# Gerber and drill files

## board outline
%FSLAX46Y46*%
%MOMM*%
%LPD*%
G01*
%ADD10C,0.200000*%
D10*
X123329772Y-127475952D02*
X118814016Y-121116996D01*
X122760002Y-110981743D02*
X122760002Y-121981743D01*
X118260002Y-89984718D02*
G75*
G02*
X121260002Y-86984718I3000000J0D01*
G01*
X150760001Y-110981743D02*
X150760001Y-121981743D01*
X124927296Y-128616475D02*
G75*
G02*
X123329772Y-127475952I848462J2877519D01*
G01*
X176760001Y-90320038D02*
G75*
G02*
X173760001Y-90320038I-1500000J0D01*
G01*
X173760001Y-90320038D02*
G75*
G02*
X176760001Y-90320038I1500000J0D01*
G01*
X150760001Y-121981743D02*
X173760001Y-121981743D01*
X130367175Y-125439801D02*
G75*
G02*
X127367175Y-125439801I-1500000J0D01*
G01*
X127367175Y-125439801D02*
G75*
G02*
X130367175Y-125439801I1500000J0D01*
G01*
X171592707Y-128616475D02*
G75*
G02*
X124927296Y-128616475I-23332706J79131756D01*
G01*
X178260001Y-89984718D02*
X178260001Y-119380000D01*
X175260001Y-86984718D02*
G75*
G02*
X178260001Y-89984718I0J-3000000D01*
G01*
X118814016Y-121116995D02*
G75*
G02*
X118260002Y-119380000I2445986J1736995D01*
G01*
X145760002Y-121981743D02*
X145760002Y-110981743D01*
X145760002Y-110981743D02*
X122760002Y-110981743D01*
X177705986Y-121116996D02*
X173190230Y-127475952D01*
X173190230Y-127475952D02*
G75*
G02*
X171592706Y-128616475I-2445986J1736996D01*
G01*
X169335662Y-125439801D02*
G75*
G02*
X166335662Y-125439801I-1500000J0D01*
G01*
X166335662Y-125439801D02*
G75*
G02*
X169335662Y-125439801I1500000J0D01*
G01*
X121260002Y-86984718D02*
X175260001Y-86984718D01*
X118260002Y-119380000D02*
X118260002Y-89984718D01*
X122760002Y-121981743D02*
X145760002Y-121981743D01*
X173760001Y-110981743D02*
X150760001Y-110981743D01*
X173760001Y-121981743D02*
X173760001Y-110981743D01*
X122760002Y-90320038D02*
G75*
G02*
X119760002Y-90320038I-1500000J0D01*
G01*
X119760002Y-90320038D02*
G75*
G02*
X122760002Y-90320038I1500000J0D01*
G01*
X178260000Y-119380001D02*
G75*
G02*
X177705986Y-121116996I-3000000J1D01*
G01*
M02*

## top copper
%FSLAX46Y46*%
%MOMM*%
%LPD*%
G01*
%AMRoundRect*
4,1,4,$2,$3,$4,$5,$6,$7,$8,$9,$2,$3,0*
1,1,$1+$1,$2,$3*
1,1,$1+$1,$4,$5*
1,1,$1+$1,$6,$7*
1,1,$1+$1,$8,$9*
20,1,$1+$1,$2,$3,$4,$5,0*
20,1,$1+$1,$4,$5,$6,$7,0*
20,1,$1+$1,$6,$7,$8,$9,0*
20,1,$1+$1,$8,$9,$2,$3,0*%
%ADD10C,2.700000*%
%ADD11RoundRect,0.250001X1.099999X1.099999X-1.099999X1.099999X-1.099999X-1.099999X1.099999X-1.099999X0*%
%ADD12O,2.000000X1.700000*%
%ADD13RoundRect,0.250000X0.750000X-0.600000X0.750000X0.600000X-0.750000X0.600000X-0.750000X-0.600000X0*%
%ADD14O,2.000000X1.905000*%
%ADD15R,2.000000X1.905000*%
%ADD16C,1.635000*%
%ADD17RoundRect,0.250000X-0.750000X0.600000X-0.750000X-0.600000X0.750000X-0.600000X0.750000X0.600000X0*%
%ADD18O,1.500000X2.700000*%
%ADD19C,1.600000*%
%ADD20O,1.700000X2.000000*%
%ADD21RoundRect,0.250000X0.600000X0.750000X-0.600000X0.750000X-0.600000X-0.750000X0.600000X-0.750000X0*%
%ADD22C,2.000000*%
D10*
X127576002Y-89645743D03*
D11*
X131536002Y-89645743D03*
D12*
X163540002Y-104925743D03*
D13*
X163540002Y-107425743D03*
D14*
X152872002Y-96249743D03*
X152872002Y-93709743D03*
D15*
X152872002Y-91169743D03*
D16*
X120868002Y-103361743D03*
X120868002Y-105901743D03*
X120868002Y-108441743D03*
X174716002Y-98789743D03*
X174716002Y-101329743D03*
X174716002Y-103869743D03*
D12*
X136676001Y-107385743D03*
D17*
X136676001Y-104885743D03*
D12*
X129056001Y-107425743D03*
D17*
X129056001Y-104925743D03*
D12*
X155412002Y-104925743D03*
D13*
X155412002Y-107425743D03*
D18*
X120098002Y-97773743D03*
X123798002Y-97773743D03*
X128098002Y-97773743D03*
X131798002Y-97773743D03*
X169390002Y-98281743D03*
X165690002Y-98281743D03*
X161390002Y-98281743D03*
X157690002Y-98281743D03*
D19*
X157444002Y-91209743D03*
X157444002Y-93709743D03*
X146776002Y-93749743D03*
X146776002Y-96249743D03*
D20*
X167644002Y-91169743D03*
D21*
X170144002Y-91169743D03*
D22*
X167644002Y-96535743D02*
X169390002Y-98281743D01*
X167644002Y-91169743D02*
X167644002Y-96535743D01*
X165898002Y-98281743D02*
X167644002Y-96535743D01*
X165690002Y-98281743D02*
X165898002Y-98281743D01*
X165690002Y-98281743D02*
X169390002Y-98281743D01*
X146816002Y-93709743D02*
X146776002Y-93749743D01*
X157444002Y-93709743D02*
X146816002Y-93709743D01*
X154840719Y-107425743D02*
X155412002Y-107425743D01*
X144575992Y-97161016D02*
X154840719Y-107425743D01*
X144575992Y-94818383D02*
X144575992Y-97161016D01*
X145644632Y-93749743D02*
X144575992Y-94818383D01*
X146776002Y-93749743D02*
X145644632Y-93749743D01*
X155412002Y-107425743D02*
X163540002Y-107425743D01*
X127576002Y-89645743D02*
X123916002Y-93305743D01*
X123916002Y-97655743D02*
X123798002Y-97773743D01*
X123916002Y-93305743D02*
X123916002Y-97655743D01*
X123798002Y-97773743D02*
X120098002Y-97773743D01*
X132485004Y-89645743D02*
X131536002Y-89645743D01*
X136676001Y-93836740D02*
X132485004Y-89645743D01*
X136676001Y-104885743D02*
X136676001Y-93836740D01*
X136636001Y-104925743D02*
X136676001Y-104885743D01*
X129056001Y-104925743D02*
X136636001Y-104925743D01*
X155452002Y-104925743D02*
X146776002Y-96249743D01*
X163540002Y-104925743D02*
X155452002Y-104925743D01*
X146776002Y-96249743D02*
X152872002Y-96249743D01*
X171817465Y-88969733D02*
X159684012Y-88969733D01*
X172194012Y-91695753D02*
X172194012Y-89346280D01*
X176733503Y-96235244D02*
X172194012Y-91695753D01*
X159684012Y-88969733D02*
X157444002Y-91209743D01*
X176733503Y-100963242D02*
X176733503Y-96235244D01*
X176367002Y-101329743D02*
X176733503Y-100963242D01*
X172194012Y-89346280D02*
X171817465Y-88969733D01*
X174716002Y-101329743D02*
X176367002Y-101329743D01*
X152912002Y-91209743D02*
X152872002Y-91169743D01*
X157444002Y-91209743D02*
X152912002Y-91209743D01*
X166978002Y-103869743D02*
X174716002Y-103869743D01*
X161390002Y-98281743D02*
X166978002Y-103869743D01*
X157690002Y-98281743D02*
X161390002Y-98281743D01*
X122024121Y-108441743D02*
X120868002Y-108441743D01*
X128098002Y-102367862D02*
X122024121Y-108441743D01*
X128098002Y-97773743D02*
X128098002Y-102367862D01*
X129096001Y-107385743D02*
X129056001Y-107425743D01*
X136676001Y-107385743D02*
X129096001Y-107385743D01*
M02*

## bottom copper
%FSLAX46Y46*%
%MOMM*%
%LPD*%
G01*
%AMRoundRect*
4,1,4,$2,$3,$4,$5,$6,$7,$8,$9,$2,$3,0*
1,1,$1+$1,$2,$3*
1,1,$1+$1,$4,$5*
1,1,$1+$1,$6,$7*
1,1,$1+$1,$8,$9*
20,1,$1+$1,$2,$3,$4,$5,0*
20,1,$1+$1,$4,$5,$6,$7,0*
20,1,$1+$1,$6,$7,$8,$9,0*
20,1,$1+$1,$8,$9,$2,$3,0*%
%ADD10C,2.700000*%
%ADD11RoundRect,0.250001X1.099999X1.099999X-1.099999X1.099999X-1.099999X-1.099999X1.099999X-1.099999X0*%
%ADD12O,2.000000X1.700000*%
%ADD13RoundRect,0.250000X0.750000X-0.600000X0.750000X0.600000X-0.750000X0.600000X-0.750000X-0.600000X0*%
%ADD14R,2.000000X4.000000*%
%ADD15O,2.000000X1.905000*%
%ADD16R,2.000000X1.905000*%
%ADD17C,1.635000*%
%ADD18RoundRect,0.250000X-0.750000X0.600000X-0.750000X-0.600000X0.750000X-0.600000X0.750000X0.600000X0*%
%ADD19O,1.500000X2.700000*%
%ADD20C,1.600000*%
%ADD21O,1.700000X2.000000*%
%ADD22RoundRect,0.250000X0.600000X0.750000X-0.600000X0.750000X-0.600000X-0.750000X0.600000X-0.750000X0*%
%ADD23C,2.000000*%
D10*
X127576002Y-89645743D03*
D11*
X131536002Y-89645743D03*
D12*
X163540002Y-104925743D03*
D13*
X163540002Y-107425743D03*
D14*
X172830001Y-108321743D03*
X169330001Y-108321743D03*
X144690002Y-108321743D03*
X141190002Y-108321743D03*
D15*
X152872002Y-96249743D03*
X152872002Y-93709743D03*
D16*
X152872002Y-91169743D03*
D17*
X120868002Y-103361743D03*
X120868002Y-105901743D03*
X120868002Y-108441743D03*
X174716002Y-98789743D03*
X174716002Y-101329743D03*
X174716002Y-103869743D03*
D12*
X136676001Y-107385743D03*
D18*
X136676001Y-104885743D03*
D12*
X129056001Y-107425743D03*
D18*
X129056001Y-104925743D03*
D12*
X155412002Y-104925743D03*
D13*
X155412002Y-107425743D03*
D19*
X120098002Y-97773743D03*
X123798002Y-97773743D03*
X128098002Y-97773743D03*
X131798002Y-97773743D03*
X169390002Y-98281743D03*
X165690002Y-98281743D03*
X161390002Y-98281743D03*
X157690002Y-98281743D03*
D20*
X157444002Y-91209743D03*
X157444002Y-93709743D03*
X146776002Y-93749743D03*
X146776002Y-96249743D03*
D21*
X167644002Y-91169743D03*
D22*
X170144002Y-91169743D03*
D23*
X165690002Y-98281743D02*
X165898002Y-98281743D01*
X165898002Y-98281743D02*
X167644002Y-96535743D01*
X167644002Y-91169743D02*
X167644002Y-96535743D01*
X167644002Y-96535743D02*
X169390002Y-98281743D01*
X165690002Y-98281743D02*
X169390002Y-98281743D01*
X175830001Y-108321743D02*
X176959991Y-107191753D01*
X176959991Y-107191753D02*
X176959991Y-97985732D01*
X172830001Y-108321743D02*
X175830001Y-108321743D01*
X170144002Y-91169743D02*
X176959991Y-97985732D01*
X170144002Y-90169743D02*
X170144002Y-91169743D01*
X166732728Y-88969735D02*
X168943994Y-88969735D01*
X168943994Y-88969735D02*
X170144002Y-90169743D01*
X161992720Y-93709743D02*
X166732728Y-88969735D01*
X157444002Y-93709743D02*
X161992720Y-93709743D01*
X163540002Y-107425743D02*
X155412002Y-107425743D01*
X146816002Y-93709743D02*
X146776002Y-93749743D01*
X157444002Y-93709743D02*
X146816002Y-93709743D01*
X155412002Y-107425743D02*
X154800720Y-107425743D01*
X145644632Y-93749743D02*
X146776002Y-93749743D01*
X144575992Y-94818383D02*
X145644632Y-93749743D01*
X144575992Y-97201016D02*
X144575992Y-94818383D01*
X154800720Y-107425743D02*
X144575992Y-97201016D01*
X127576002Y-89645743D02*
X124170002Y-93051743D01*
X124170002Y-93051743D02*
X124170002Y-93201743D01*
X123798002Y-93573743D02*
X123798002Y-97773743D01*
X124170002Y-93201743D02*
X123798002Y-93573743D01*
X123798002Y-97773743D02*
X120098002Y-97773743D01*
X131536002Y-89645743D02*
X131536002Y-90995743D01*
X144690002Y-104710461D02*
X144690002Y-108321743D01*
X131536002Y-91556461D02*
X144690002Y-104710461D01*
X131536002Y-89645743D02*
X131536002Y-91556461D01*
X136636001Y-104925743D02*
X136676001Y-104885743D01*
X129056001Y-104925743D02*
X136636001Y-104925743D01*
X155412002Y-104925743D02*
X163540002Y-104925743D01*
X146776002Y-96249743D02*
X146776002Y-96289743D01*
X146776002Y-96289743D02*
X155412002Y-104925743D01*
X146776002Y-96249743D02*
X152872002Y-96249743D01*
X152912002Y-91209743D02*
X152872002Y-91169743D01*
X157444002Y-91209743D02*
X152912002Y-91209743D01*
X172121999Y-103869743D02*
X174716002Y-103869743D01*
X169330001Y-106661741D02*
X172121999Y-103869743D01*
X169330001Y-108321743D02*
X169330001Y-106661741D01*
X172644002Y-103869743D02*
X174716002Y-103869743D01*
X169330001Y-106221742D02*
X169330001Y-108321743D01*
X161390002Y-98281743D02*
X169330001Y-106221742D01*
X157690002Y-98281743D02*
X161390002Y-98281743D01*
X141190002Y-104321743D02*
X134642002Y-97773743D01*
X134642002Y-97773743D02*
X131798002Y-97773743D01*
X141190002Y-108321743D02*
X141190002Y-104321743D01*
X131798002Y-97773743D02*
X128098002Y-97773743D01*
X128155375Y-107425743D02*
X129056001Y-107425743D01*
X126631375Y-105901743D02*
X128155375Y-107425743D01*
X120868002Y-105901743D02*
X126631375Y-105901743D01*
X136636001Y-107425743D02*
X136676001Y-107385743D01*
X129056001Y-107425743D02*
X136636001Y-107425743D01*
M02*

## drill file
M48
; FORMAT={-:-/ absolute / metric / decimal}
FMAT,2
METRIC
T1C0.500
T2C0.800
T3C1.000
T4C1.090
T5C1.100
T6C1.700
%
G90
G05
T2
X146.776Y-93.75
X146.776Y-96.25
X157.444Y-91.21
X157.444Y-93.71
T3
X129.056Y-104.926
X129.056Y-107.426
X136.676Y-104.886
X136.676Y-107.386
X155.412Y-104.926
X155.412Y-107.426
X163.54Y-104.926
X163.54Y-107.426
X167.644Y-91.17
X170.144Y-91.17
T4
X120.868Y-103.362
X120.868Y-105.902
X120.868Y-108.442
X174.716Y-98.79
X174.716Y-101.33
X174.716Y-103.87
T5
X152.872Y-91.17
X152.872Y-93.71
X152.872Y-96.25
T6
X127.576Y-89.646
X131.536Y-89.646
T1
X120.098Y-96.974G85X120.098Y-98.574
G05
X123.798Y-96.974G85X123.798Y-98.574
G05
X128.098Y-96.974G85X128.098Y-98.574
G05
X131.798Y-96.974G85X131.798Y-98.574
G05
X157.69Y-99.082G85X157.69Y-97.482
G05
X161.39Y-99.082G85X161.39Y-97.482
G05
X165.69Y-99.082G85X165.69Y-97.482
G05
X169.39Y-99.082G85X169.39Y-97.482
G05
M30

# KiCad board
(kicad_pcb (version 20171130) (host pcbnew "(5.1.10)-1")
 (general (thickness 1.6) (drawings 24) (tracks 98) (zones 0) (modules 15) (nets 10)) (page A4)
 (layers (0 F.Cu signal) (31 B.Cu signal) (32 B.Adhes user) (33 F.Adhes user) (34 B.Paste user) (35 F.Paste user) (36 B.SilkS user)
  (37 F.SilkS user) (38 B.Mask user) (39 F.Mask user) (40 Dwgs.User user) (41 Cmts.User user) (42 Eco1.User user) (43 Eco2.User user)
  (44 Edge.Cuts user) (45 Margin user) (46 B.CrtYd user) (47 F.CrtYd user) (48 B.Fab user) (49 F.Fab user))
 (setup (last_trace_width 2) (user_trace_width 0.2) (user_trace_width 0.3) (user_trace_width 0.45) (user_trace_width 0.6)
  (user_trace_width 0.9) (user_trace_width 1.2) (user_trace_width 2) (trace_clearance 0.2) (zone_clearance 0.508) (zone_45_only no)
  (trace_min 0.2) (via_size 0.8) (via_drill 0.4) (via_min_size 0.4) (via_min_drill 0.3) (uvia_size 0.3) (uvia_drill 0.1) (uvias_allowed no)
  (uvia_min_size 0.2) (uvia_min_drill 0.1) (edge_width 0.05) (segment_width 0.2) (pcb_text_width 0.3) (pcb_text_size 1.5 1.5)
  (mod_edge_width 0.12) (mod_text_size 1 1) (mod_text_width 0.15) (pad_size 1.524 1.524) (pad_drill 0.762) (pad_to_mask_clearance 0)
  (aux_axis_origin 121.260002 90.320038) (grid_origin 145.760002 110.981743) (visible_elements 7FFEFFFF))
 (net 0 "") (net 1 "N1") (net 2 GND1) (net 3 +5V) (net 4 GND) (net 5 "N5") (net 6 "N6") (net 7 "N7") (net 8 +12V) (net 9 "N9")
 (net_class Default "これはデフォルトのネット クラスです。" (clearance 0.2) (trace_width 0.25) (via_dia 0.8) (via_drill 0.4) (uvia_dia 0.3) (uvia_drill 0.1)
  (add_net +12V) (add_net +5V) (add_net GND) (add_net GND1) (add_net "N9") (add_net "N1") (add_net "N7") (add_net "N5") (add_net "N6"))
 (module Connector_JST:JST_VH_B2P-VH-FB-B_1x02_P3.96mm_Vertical (layer F.Cu) (at 131.536002 89.645743 180)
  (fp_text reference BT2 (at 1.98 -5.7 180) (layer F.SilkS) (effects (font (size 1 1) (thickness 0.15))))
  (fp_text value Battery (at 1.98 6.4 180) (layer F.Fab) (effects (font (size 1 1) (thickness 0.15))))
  (pad 2 thru_hole circle (at 3.96 0 180) (size 2.7 2.7) (drill 1.7) (layers *.Cu *.Mask) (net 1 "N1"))
  (pad 1 thru_hole roundrect (at 0 0 180) (size 2.7 2.7) (drill 1.7) (layers *.Cu *.Mask) (roundrect_rratio 0.09259299999999999)
   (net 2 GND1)))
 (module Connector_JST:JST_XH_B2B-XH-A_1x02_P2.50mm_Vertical (layer F.Cu) (at 163.540002 107.425743 90)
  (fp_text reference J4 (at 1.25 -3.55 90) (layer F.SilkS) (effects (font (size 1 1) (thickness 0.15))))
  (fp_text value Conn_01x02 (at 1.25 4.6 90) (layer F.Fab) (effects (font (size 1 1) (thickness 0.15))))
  (pad 2 thru_hole oval (at 2.5 0 90) (size 1.7 2) (drill 1) (layers *.Cu *.Mask) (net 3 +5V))
  (pad 1 thru_hole roundrect (at 0 0 90) (size 1.7 2) (drill 1) (layers *.Cu *.Mask) (roundrect_rratio 0.147059) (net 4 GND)))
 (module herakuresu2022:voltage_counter (layer F.Cu) (at 162.330001 111.821743)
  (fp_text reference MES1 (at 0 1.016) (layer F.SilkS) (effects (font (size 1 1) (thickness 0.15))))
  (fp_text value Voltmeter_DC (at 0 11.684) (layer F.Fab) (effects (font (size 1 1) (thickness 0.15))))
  (pad 1 smd rect (at 10.5 -3.5) (size 2 4) (layers B.Cu B.Paste B.Mask) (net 4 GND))
  (pad 2 smd rect (at 7 -3.5) (size 2 4) (layers B.Cu B.Paste B.Mask) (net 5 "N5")))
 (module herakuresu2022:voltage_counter (layer F.Cu) (at 134.190002 111.821743)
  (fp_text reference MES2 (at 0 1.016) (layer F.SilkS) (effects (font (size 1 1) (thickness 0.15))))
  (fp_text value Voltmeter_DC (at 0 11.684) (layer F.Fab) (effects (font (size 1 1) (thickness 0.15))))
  (pad 1 smd rect (at 10.5 -3.5) (size 2 4) (layers B.Cu B.Paste B.Mask) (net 2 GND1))
  (pad 2 smd rect (at 7 -3.5) (size 2 4) (layers B.Cu B.Paste B.Mask) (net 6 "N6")))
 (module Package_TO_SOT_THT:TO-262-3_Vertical (layer F.Cu) (at 152.872002 91.169743 270)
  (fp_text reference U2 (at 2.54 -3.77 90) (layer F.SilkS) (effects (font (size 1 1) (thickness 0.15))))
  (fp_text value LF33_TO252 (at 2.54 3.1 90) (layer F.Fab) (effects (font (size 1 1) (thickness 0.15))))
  (pad 3 thru_hole oval (at 5.08 0 270) (size 1.905 2) (drill 1.1) (layers *.Cu *.Mask) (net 3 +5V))
  (pad 2 thru_hole oval (at 2.54 0 270) (size 1.905 2) (drill 1.1) (layers *.Cu *.Mask) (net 4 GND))
  (pad 1 thru_hole rect (at 0 0 270) (size 1.905 2) (drill 1.1) (layers *.Cu *.Mask) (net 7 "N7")))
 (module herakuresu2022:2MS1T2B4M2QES (layer F.Cu) (at 120.868002 108.441743)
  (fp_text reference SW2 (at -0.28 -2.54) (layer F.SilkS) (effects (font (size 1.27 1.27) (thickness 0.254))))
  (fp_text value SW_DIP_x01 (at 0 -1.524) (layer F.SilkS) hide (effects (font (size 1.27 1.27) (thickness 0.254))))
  (pad 3 thru_hole circle (at 0 -5.08) (size 1.635 1.635) (drill 1.09) (layers *.Cu *.Mask))
  (pad 2 thru_hole circle (at 0 -2.54) (size 1.635 1.635) (drill 1.09) (layers *.Cu *.Mask) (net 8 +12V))
  (pad 1 thru_hole circle (at 0 0) (size 1.635 1.635) (drill 1.09) (layers *.Cu *.Mask) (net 6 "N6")))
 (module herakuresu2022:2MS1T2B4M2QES (layer F.Cu) (at 174.716002 103.869743)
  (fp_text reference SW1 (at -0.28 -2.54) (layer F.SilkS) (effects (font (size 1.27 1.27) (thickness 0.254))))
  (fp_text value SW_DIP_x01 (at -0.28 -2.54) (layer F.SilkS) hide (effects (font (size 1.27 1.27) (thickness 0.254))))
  (pad 3 thru_hole circle (at 0 -5.08) (size 1.635 1.635) (drill 1.09) (layers *.Cu *.Mask))
  (pad 2 thru_hole circle (at 0 -2.54) (size 1.635 1.635) (drill 1.09) (layers *.Cu *.Mask) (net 7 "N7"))
  (pad 1 thru_hole circle (at 0 0) (size 1.635 1.635) (drill 1.09) (layers *.Cu *.Mask) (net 5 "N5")))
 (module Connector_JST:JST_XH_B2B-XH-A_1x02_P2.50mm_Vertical (layer F.Cu) (at 136.676001 104.885743 270)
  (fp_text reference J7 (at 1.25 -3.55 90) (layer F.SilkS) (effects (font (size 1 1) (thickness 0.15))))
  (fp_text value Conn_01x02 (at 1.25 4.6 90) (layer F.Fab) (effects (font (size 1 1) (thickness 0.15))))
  (pad 2 thru_hole oval (at 2.5 0 270) (size 1.7 2) (drill 1) (layers *.Cu *.Mask) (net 8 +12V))
  (pad 1 thru_hole roundrect (at 0 0 270) (size 1.7 2) (drill 1) (layers *.Cu *.Mask) (roundrect_rratio 0.147059) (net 2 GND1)))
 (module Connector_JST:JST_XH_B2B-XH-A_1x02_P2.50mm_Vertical (layer F.Cu) (at 129.056001 104.925743 270)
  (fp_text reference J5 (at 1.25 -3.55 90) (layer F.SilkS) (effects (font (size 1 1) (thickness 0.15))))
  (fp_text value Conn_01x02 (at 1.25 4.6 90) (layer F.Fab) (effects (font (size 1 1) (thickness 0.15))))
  (pad 2 thru_hole oval (at 2.5 0 270) (size 1.7 2) (drill 1) (layers *.Cu *.Mask) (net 8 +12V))
  (pad 1 thru_hole roundrect (at 0 0 270) (size 1.7 2) (drill 1) (layers *.Cu *.Mask) (roundrect_rratio 0.147059) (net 2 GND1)))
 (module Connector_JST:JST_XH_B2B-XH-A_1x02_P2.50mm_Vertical (layer F.Cu) (at 155.412002 107.425743 90)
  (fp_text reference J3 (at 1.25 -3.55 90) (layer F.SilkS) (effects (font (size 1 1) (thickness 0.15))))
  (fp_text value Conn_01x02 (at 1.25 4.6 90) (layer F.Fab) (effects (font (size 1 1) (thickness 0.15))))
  (pad 2 thru_hole oval (at 2.5 0 90) (size 1.7 2) (drill 1) (layers *.Cu *.Mask) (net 3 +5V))
  (pad 1 thru_hole roundrect (at 0 0 90) (size 1.7 2) (drill 1) (layers *.Cu *.Mask) (roundrect_rratio 0.147059) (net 4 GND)))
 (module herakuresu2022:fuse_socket (layer F.Cu) (at 125.948002 95.233743)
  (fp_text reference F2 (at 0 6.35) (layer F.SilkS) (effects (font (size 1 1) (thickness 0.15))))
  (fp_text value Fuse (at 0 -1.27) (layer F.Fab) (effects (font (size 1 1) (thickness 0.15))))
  (pad 1 thru_hole oval (at -5.85 2.54) (size 1.5 2.7) (drill oval 0.5 2.1) (layers *.Cu *.Mask) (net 1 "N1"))
  (pad 1 thru_hole oval (at -2.15 2.54) (size 1.5 2.7) (drill oval 0.5 2.1) (layers *.Cu *.Mask) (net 1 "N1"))
  (pad 2 thru_hole oval (at 2.15 2.54) (size 1.5 2.7) (drill oval 0.5 2.1) (layers *.Cu *.Mask) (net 6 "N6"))
  (pad 2 thru_hole oval (at 5.85 2.54) (size 1.5 2.7) (drill oval 0.5 2.1) (layers *.Cu *.Mask) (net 6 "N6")))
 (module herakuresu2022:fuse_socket (layer F.Cu) (at 163.540002 100.821743 180)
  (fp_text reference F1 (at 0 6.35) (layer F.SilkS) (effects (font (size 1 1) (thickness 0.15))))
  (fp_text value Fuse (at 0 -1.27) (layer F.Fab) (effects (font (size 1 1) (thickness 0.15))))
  (pad 1 thru_hole oval (at -5.85 2.54 180) (size 1.5 2.7) (drill oval 0.5 2.1) (layers *.Cu *.Mask) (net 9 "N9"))
  (pad 1 thru_hole oval (at -2.15 2.54 180) (size 1.5 2.7) (drill oval 0.5 2.1) (layers *.Cu *.Mask) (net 9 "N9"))
  (pad 2 thru_hole oval (at 2.15 2.54 180) (size 1.5 2.7) (drill oval 0.5 2.1) (layers *.Cu *.Mask) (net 5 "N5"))
  (pad 2 thru_hole oval (at 5.85 2.54 180) (size 1.5 2.7) (drill oval 0.5 2.1) (layers *.Cu *.Mask) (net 5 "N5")))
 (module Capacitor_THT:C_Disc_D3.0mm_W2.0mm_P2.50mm (layer F.Cu) (at 157.444002 93.709743 90)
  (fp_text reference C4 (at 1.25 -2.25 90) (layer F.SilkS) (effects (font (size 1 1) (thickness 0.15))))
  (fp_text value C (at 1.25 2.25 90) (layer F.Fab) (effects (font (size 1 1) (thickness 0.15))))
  (pad 2 thru_hole circle (at 2.5 0 90) (size 1.6 1.6) (drill 0.8) (layers *.Cu *.Mask) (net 7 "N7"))
  (pad 1 thru_hole circle (at 0 0 90) (size 1.6 1.6) (drill 0.8) (layers *.Cu *.Mask) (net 4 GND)))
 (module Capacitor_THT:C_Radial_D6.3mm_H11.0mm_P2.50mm (layer F.Cu) (at 146.776002 96.249743 90)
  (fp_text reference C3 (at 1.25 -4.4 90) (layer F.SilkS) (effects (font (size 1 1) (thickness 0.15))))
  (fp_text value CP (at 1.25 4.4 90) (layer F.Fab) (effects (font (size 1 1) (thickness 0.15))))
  (pad 2 thru_hole circle (at 2.5 0 90) (size 1.6 1.6) (drill 0.8) (layers *.Cu *.Mask) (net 4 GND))
  (pad 1 thru_hole circle (at 0 0 90) (size 1.6 1.6) (drill 0.8) (layers *.Cu *.Mask) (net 3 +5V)))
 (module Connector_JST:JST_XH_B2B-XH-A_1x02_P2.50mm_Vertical (layer F.Cu) (at 170.144002 91.169743 180)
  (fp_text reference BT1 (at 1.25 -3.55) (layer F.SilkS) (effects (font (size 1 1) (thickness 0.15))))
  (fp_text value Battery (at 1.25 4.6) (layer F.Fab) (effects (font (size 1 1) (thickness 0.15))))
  (pad 2 thru_hole oval (at 2.5 0 180) (size 1.7 2) (drill 1) (layers *.Cu *.Mask) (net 9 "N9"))
  (pad 1 thru_hole roundrect (at 0 0 180) (size 1.7 2) (drill 1) (layers *.Cu *.Mask) (roundrect_rratio 0.147059) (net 4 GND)))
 (gr_line (start 123.329772 127.475952) (end 118.814016 121.116996) (layer Edge.Cuts) (width 0.2))
 (gr_line (start 122.760002 110.981743) (end 122.760002 121.981743) (layer Edge.Cuts) (width 0.2))
 (gr_arc (start 121.260002 89.984718) (end 121.260002 86.984718) (angle -90) (layer Edge.Cuts) (width 0.2))
 (gr_line (start 150.760001 110.981743) (end 150.760001 121.981743) (layer Edge.Cuts) (width 0.2))
 (gr_arc (start 125.775758 125.738956) (end 123.329772 127.475952) (angle -38.19124813) (layer Edge.Cuts) (width 0.2))
 (gr_circle (center 175.260001 90.320038) (end 173.760001 90.320038) (layer Edge.Cuts) (width 0.2))
 (gr_line (start 150.760001 121.981743) (end 173.760001 121.981743) (layer Edge.Cuts) (width 0.2))
 (gr_circle (center 128.867175 125.439801) (end 127.367175 125.439801) (layer Edge.Cuts) (width 0.2))
 (gr_arc (start 148.260001 49.484719) (end 124.927296 128.616475) (angle -32.85724767) (layer Edge.Cuts) (width 0.2))
 (gr_line (start 178.260001 89.984718) (end 178.260001 119.38) (layer Edge.Cuts) (width 0.2))
 (gr_arc (start 175.260001 89.984718) (end 178.260001 89.984718) (angle -90) (layer Edge.Cuts) (width 0.2))
 (gr_arc (start 121.260002 119.38) (end 118.260002 119.38) (angle -35.38012804) (layer Edge.Cuts) (width 0.2))
 (gr_line (start 145.760002 121.981743) (end 145.760002 110.981743) (layer Edge.Cuts) (width 0.2))
 (gr_line (start 145.760002 110.981743) (end 122.760002 110.981743) (layer Edge.Cuts) (width 0.2))
 (gr_line (start 177.705986 121.116996) (end 173.19023 127.475952) (layer Edge.Cuts) (width 0.2))
 (gr_arc (start 170.744244 125.738956) (end 171.592706 128.616475) (angle -38.19124813) (layer Edge.Cuts) (width 0.2))
 (gr_circle (center 167.835662 125.439801) (end 166.335662 125.439801) (layer Edge.Cuts) (width 0.2))
 (gr_line (start 121.260002 86.984718) (end 175.260001 86.984718) (layer Edge.Cuts) (width 0.2))
 (gr_line (start 118.260002 119.38) (end 118.260002 89.984718) (layer Edge.Cuts) (width 0.2))
 (gr_line (start 122.760002 121.981743) (end 145.760002 121.981743) (layer Edge.Cuts) (width 0.2))
 (gr_line (start 173.760001 110.981743) (end 150.760001 110.981743) (layer Edge.Cuts) (width 0.2))
 (gr_line (start 173.760001 121.981743) (end 173.760001 110.981743) (layer Edge.Cuts) (width 0.2))
 (gr_circle (center 121.260002 90.320038) (end 119.760002 90.320038) (layer Edge.Cuts) (width 0.2))
 (gr_arc (start 175.26 119.38) (end 177.705986 121.116996) (angle -35.38012804) (layer Edge.Cuts) (width 0.2))
 (segment (start 165.690002 98.281743) (end 165.898002 98.281743) (width 2) (layer B.Cu) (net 9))
 (segment (start 165.898002 98.281743) (end 167.644002 96.535743) (width 2) (layer B.Cu) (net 9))
 (segment (start 167.644002 91.169743) (end 167.644002 96.535743) (width 2) (layer B.Cu) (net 9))
 (segment (start 167.644002 96.535743) (end 169.390002 98.281743) (width 2) (layer B.Cu) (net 9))
 (segment (start 167.644002 96.535743) (end 169.390002 98.281743) (width 2) (layer F.Cu) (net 9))
 (segment (start 167.644002 91.169743) (end 167.644002 96.535743) (width 2) (layer F.Cu) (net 9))
 (segment (start 165.898002 98.281743) (end 167.644002 96.535743) (width 2) (layer F.Cu) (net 9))
 (segment (start 165.690002 98.281743) (end 165.898002 98.281743) (width 2) (layer F.Cu) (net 9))
 (segment (start 165.690002 98.281743) (end 169.390002 98.281743) (width 2) (layer B.Cu) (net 9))
 (segment (start 165.690002 98.281743) (end 169.390002 98.281743) (width 2) (layer F.Cu) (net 9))
 (segment (start 175.830001 108.321743) (end 176.959991 107.191753) (width 2) (layer B.Cu) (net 4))
 (segment (start 176.959991 107.191753) (end 176.959991 97.985732) (width 2) (layer B.Cu) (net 4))
 (segment (start 172.830001 108.321743) (end 175.830001 108.321743) (width 2) (layer B.Cu) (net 4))
 (segment (start 170.144002 91.169743) (end 176.959991 97.985732) (width 2) (layer B.Cu) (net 4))
 (segment (start 170.144002 90.169743) (end 170.144002 91.169743) (width 2) (layer B.Cu) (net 4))
 (segment (start 166.732728 88.969735) (end 168.943994 88.969735) (width 2) (layer B.Cu) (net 4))
 (segment (start 168.943994 88.969735) (end 170.144002 90.169743) (width 2) (layer B.Cu) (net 4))
 (segment (start 161.99272 93.709743) (end 166.732728 88.969735) (width 2) (layer B.Cu) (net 4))
 (segment (start 157.444002 93.709743) (end 161.99272 93.709743) (width 2) (layer B.Cu) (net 4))
 (segment (start 146.816002 93.709743) (end 146.776002 93.749743) (width 2) (layer F.Cu) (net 4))
 (segment (start 157.444002 93.709743) (end 146.816002 93.709743) (width 2) (layer F.Cu) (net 4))
 (segment (start 154.840719 107.425743) (end 155.412002 107.425743) (width 2) (layer F.Cu) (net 4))
 (segment (start 144.575992 97.161016) (end 154.840719 107.425743) (width 2) (layer F.Cu) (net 4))
 (segment (start 144.575992 94.818383) (end 144.575992 97.161016) (width 2) (layer F.Cu) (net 4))
 (segment (start 145.644632 93.749743) (end 144.575992 94.818383) (width 2) (layer F.Cu) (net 4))
 (segment (start 146.776002 93.749743) (end 145.644632 93.749743) (width 2) (layer F.Cu) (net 4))
 (segment (start 163.540002 107.425743) (end 155.412002 107.425743) (width 2) (layer B.Cu) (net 4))
 (segment (start 155.412002 107.425743) (end 163.540002 107.425743) (width 2) (layer F.Cu) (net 4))
 (segment (start 146.816002 93.709743) (end 146.776002 93.749743) (width 2) (layer B.Cu) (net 4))
 (segment (start 157.444002 93.709743) (end 146.816002 93.709743) (width 2) (layer B.Cu) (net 4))
 (segment (start 155.412002 107.425743) (end 154.80072 107.425743) (width 2) (layer B.Cu) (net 4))
 (segment (start 145.644632 93.749743) (end 146.776002 93.749743) (width 2) (layer B.Cu) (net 4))
 (segment (start 144.575992 94.818383) (end 145.644632 93.749743) (width 2) (layer B.Cu) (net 4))
 (segment (start 144.575992 97.201016) (end 144.575992 94.818383) (width 2) (layer B.Cu) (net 4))
 (segment (start 154.80072 107.425743) (end 144.575992 97.201016) (width 2) (layer B.Cu) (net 4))
 (segment (start 127.576002 89.645743) (end 123.916002 93.305743) (width 2) (layer F.Cu) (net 1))
 (segment (start 123.916002 97.655743) (end 123.798002 97.773743) (width 2) (layer F.Cu) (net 1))
 (segment (start 123.916002 93.305743) (end 123.916002 97.655743) (width 2) (layer F.Cu) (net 1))
 (segment (start 123.798002 97.773743) (end 120.098002 97.773743) (width 2) (layer F.Cu) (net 1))
 (segment (start 127.576002 89.645743) (end 124.170002 93.051743) (width 2) (layer B.Cu) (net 1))
 (segment (start 124.170002 93.051743) (end 124.170002 93.201743) (width 2) (layer B.Cu) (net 1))
 (segment (start 123.798002 93.573743) (end 123.798002 97.773743) (width 2) (layer B.Cu) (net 1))
 (segment (start 124.170002 93.201743) (end 123.798002 93.573743) (width 2) (layer B.Cu) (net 1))
 (segment (start 123.798002 97.773743) (end 120.098002 97.773743) (width 2) (layer B.Cu) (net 1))
 (segment (start 132.485004 89.645743) (end 131.536002 89.645743) (width 2) (layer F.Cu) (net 2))
 (segment (start 136.676001 93.83674) (end 132.485004 89.645743) (width 2) (layer F.Cu) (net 2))
 (segment (start 136.676001 104.885743) (end 136.676001 93.83674) (width 2) (layer F.Cu) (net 2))
 (segment (start 131.536002 89.645743) (end 131.536002 90.995743) (width 2) (layer B.Cu) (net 2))
 (segment (start 144.690002 104.710461) (end 144.690002 108.321743) (width 2) (layer B.Cu) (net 2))
 (segment (start 131.536002 91.556461) (end 144.690002 104.710461) (width 2) (layer B.Cu) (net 2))
 (segment (start 131.536002 89.645743) (end 131.536002 91.556461) (width 2) (layer B.Cu) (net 2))
 (segment (start 136.636001 104.925743) (end 136.676001 104.885743) (width 2) (layer F.Cu) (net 2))
 (segment (start 129.056001 104.925743) (end 136.636001 104.925743) (width 2) (layer F.Cu) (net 2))
 (segment (start 136.636001 104.925743) (end 136.676001 104.885743) (width 2) (layer B.Cu) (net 2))
 (segment (start 129.056001 104.925743) (end 136.636001 104.925743) (width 2) (layer B.Cu) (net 2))
 (segment (start 155.412002 104.925743) (end 163.540002 104.925743) (width 2) (layer B.Cu) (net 3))
 (segment (start 146.776002 96.249743) (end 146.776002 96.289743) (width 2) (layer B.Cu) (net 3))
 (segment (start 146.776002 96.289743) (end 155.412002 104.925743) (width 2) (layer B.Cu) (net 3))
 (segment (start 155.452002 104.925743) (end 146.776002 96.249743) (width 2) (layer F.Cu) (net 3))
 (segment (start 163.540002 104.925743) (end 155.452002 104.925743) (width 2) (layer F.Cu) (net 3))
 (segment (start 146.776002 96.249743) (end 152.872002 96.249743) (width 2) (layer B.Cu) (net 3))
 (segment (start 146.776002 96.249743) (end 152.872002 96.249743) (width 2) (layer F.Cu) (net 3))
 (segment (start 171.817465 88.969733) (end 159.684012 88.969733) (width 2) (layer F.Cu) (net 7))
 (segment (start 172.194012 91.695753) (end 172.194012 89.34628) (width 2) (layer F.Cu) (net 7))
 (segment (start 176.733503 96.235244) (end 172.194012 91.695753) (width 2) (layer F.Cu) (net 7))
 (segment (start 159.684012 88.969733) (end 157.444002 91.209743) (width 2) (layer F.Cu) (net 7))
 (segment (start 176.733503 100.963242) (end 176.733503 96.235244) (width 2) (layer F.Cu) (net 7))
 (segment (start 176.367002 101.329743) (end 176.733503 100.963242) (width 2) (layer F.Cu) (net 7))
 (segment (start 172.194012 89.34628) (end 171.817465 88.969733) (width 2) (layer F.Cu) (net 7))
 (segment (start 174.716002 101.329743) (end 176.367002 101.329743) (width 2) (layer F.Cu) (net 7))
 (segment (start 152.912002 91.209743) (end 152.872002 91.169743) (width 2) (layer F.Cu) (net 7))
 (segment (start 157.444002 91.209743) (end 152.912002 91.209743) (width 2) (layer F.Cu) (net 7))
 (segment (start 152.912002 91.209743) (end 152.872002 91.169743) (width 2) (layer B.Cu) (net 7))
 (segment (start 157.444002 91.209743) (end 152.912002 91.209743) (width 2) (layer B.Cu) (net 7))
 (segment (start 172.121999 103.869743) (end 174.716002 103.869743) (width 2) (layer B.Cu) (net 5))
 (segment (start 169.330001 106.661741) (end 172.121999 103.869743) (width 2) (layer B.Cu) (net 5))
 (segment (start 169.330001 108.321743) (end 169.330001 106.661741) (width 2) (layer B.Cu) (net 5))
 (segment (start 172.644002 103.869743) (end 174.716002 103.869743) (width 2) (layer B.Cu) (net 5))
 (segment (start 169.330001 106.221742) (end 169.330001 108.321743) (width 2) (layer B.Cu) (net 5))
 (segment (start 161.390002 98.281743) (end 169.330001 106.221742) (width 2) (layer B.Cu) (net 5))
 (segment (start 166.978002 103.869743) (end 174.716002 103.869743) (width 2) (layer F.Cu) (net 5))
 (segment (start 161.390002 98.281743) (end 166.978002 103.869743) (width 2) (layer F.Cu) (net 5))
 (segment (start 157.690002 98.281743) (end 161.390002 98.281743) (width 2) (layer B.Cu) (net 5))
 (segment (start 157.690002 98.281743) (end 161.390002 98.281743) (width 2) (layer F.Cu) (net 5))
 (segment (start 141.190002 104.321743) (end 134.642002 97.773743) (width 2) (layer B.Cu) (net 6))
 (segment (start 134.642002 97.773743) (end 131.798002 97.773743) (width 2) (layer B.Cu) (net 6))
 (segment (start 141.190002 108.321743) (end 141.190002 104.321743) (width 2) (layer B.Cu) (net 6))
 (segment (start 131.798002 97.773743) (end 128.098002 97.773743) (width 2) (layer B.Cu) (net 6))
 (segment (start 122.024121 108.441743) (end 120.868002 108.441743) (width 2) (layer F.Cu) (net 6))
 (segment (start 128.098002 102.367862) (end 122.024121 108.441743) (width 2) (layer F.Cu) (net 6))
 (segment (start 128.098002 97.773743) (end 128.098002 102.367862) (width 2) (layer F.Cu) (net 6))
 (segment (start 128.155375 107.425743) (end 129.056001 107.425743) (width 2) (layer B.Cu) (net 8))
 (segment (start 126.631375 105.901743) (end 128.155375 107.425743) (width 2) (layer B.Cu) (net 8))
 (segment (start 120.868002 105.901743) (end 126.631375 105.901743) (width 2) (layer B.Cu) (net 8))
 (segment (start 129.096001 107.385743) (end 129.056001 107.425743) (width 2) (layer F.Cu) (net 8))
 (segment (start 136.676001 107.385743) (end 129.096001 107.385743) (width 2) (layer F.Cu) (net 8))
 (segment (start 136.636001 107.425743) (end 136.676001 107.385743) (width 2) (layer B.Cu) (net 8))
 (segment (start 129.056001 107.425743) (end 136.636001 107.425743) (width 2) (layer B.Cu) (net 8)))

